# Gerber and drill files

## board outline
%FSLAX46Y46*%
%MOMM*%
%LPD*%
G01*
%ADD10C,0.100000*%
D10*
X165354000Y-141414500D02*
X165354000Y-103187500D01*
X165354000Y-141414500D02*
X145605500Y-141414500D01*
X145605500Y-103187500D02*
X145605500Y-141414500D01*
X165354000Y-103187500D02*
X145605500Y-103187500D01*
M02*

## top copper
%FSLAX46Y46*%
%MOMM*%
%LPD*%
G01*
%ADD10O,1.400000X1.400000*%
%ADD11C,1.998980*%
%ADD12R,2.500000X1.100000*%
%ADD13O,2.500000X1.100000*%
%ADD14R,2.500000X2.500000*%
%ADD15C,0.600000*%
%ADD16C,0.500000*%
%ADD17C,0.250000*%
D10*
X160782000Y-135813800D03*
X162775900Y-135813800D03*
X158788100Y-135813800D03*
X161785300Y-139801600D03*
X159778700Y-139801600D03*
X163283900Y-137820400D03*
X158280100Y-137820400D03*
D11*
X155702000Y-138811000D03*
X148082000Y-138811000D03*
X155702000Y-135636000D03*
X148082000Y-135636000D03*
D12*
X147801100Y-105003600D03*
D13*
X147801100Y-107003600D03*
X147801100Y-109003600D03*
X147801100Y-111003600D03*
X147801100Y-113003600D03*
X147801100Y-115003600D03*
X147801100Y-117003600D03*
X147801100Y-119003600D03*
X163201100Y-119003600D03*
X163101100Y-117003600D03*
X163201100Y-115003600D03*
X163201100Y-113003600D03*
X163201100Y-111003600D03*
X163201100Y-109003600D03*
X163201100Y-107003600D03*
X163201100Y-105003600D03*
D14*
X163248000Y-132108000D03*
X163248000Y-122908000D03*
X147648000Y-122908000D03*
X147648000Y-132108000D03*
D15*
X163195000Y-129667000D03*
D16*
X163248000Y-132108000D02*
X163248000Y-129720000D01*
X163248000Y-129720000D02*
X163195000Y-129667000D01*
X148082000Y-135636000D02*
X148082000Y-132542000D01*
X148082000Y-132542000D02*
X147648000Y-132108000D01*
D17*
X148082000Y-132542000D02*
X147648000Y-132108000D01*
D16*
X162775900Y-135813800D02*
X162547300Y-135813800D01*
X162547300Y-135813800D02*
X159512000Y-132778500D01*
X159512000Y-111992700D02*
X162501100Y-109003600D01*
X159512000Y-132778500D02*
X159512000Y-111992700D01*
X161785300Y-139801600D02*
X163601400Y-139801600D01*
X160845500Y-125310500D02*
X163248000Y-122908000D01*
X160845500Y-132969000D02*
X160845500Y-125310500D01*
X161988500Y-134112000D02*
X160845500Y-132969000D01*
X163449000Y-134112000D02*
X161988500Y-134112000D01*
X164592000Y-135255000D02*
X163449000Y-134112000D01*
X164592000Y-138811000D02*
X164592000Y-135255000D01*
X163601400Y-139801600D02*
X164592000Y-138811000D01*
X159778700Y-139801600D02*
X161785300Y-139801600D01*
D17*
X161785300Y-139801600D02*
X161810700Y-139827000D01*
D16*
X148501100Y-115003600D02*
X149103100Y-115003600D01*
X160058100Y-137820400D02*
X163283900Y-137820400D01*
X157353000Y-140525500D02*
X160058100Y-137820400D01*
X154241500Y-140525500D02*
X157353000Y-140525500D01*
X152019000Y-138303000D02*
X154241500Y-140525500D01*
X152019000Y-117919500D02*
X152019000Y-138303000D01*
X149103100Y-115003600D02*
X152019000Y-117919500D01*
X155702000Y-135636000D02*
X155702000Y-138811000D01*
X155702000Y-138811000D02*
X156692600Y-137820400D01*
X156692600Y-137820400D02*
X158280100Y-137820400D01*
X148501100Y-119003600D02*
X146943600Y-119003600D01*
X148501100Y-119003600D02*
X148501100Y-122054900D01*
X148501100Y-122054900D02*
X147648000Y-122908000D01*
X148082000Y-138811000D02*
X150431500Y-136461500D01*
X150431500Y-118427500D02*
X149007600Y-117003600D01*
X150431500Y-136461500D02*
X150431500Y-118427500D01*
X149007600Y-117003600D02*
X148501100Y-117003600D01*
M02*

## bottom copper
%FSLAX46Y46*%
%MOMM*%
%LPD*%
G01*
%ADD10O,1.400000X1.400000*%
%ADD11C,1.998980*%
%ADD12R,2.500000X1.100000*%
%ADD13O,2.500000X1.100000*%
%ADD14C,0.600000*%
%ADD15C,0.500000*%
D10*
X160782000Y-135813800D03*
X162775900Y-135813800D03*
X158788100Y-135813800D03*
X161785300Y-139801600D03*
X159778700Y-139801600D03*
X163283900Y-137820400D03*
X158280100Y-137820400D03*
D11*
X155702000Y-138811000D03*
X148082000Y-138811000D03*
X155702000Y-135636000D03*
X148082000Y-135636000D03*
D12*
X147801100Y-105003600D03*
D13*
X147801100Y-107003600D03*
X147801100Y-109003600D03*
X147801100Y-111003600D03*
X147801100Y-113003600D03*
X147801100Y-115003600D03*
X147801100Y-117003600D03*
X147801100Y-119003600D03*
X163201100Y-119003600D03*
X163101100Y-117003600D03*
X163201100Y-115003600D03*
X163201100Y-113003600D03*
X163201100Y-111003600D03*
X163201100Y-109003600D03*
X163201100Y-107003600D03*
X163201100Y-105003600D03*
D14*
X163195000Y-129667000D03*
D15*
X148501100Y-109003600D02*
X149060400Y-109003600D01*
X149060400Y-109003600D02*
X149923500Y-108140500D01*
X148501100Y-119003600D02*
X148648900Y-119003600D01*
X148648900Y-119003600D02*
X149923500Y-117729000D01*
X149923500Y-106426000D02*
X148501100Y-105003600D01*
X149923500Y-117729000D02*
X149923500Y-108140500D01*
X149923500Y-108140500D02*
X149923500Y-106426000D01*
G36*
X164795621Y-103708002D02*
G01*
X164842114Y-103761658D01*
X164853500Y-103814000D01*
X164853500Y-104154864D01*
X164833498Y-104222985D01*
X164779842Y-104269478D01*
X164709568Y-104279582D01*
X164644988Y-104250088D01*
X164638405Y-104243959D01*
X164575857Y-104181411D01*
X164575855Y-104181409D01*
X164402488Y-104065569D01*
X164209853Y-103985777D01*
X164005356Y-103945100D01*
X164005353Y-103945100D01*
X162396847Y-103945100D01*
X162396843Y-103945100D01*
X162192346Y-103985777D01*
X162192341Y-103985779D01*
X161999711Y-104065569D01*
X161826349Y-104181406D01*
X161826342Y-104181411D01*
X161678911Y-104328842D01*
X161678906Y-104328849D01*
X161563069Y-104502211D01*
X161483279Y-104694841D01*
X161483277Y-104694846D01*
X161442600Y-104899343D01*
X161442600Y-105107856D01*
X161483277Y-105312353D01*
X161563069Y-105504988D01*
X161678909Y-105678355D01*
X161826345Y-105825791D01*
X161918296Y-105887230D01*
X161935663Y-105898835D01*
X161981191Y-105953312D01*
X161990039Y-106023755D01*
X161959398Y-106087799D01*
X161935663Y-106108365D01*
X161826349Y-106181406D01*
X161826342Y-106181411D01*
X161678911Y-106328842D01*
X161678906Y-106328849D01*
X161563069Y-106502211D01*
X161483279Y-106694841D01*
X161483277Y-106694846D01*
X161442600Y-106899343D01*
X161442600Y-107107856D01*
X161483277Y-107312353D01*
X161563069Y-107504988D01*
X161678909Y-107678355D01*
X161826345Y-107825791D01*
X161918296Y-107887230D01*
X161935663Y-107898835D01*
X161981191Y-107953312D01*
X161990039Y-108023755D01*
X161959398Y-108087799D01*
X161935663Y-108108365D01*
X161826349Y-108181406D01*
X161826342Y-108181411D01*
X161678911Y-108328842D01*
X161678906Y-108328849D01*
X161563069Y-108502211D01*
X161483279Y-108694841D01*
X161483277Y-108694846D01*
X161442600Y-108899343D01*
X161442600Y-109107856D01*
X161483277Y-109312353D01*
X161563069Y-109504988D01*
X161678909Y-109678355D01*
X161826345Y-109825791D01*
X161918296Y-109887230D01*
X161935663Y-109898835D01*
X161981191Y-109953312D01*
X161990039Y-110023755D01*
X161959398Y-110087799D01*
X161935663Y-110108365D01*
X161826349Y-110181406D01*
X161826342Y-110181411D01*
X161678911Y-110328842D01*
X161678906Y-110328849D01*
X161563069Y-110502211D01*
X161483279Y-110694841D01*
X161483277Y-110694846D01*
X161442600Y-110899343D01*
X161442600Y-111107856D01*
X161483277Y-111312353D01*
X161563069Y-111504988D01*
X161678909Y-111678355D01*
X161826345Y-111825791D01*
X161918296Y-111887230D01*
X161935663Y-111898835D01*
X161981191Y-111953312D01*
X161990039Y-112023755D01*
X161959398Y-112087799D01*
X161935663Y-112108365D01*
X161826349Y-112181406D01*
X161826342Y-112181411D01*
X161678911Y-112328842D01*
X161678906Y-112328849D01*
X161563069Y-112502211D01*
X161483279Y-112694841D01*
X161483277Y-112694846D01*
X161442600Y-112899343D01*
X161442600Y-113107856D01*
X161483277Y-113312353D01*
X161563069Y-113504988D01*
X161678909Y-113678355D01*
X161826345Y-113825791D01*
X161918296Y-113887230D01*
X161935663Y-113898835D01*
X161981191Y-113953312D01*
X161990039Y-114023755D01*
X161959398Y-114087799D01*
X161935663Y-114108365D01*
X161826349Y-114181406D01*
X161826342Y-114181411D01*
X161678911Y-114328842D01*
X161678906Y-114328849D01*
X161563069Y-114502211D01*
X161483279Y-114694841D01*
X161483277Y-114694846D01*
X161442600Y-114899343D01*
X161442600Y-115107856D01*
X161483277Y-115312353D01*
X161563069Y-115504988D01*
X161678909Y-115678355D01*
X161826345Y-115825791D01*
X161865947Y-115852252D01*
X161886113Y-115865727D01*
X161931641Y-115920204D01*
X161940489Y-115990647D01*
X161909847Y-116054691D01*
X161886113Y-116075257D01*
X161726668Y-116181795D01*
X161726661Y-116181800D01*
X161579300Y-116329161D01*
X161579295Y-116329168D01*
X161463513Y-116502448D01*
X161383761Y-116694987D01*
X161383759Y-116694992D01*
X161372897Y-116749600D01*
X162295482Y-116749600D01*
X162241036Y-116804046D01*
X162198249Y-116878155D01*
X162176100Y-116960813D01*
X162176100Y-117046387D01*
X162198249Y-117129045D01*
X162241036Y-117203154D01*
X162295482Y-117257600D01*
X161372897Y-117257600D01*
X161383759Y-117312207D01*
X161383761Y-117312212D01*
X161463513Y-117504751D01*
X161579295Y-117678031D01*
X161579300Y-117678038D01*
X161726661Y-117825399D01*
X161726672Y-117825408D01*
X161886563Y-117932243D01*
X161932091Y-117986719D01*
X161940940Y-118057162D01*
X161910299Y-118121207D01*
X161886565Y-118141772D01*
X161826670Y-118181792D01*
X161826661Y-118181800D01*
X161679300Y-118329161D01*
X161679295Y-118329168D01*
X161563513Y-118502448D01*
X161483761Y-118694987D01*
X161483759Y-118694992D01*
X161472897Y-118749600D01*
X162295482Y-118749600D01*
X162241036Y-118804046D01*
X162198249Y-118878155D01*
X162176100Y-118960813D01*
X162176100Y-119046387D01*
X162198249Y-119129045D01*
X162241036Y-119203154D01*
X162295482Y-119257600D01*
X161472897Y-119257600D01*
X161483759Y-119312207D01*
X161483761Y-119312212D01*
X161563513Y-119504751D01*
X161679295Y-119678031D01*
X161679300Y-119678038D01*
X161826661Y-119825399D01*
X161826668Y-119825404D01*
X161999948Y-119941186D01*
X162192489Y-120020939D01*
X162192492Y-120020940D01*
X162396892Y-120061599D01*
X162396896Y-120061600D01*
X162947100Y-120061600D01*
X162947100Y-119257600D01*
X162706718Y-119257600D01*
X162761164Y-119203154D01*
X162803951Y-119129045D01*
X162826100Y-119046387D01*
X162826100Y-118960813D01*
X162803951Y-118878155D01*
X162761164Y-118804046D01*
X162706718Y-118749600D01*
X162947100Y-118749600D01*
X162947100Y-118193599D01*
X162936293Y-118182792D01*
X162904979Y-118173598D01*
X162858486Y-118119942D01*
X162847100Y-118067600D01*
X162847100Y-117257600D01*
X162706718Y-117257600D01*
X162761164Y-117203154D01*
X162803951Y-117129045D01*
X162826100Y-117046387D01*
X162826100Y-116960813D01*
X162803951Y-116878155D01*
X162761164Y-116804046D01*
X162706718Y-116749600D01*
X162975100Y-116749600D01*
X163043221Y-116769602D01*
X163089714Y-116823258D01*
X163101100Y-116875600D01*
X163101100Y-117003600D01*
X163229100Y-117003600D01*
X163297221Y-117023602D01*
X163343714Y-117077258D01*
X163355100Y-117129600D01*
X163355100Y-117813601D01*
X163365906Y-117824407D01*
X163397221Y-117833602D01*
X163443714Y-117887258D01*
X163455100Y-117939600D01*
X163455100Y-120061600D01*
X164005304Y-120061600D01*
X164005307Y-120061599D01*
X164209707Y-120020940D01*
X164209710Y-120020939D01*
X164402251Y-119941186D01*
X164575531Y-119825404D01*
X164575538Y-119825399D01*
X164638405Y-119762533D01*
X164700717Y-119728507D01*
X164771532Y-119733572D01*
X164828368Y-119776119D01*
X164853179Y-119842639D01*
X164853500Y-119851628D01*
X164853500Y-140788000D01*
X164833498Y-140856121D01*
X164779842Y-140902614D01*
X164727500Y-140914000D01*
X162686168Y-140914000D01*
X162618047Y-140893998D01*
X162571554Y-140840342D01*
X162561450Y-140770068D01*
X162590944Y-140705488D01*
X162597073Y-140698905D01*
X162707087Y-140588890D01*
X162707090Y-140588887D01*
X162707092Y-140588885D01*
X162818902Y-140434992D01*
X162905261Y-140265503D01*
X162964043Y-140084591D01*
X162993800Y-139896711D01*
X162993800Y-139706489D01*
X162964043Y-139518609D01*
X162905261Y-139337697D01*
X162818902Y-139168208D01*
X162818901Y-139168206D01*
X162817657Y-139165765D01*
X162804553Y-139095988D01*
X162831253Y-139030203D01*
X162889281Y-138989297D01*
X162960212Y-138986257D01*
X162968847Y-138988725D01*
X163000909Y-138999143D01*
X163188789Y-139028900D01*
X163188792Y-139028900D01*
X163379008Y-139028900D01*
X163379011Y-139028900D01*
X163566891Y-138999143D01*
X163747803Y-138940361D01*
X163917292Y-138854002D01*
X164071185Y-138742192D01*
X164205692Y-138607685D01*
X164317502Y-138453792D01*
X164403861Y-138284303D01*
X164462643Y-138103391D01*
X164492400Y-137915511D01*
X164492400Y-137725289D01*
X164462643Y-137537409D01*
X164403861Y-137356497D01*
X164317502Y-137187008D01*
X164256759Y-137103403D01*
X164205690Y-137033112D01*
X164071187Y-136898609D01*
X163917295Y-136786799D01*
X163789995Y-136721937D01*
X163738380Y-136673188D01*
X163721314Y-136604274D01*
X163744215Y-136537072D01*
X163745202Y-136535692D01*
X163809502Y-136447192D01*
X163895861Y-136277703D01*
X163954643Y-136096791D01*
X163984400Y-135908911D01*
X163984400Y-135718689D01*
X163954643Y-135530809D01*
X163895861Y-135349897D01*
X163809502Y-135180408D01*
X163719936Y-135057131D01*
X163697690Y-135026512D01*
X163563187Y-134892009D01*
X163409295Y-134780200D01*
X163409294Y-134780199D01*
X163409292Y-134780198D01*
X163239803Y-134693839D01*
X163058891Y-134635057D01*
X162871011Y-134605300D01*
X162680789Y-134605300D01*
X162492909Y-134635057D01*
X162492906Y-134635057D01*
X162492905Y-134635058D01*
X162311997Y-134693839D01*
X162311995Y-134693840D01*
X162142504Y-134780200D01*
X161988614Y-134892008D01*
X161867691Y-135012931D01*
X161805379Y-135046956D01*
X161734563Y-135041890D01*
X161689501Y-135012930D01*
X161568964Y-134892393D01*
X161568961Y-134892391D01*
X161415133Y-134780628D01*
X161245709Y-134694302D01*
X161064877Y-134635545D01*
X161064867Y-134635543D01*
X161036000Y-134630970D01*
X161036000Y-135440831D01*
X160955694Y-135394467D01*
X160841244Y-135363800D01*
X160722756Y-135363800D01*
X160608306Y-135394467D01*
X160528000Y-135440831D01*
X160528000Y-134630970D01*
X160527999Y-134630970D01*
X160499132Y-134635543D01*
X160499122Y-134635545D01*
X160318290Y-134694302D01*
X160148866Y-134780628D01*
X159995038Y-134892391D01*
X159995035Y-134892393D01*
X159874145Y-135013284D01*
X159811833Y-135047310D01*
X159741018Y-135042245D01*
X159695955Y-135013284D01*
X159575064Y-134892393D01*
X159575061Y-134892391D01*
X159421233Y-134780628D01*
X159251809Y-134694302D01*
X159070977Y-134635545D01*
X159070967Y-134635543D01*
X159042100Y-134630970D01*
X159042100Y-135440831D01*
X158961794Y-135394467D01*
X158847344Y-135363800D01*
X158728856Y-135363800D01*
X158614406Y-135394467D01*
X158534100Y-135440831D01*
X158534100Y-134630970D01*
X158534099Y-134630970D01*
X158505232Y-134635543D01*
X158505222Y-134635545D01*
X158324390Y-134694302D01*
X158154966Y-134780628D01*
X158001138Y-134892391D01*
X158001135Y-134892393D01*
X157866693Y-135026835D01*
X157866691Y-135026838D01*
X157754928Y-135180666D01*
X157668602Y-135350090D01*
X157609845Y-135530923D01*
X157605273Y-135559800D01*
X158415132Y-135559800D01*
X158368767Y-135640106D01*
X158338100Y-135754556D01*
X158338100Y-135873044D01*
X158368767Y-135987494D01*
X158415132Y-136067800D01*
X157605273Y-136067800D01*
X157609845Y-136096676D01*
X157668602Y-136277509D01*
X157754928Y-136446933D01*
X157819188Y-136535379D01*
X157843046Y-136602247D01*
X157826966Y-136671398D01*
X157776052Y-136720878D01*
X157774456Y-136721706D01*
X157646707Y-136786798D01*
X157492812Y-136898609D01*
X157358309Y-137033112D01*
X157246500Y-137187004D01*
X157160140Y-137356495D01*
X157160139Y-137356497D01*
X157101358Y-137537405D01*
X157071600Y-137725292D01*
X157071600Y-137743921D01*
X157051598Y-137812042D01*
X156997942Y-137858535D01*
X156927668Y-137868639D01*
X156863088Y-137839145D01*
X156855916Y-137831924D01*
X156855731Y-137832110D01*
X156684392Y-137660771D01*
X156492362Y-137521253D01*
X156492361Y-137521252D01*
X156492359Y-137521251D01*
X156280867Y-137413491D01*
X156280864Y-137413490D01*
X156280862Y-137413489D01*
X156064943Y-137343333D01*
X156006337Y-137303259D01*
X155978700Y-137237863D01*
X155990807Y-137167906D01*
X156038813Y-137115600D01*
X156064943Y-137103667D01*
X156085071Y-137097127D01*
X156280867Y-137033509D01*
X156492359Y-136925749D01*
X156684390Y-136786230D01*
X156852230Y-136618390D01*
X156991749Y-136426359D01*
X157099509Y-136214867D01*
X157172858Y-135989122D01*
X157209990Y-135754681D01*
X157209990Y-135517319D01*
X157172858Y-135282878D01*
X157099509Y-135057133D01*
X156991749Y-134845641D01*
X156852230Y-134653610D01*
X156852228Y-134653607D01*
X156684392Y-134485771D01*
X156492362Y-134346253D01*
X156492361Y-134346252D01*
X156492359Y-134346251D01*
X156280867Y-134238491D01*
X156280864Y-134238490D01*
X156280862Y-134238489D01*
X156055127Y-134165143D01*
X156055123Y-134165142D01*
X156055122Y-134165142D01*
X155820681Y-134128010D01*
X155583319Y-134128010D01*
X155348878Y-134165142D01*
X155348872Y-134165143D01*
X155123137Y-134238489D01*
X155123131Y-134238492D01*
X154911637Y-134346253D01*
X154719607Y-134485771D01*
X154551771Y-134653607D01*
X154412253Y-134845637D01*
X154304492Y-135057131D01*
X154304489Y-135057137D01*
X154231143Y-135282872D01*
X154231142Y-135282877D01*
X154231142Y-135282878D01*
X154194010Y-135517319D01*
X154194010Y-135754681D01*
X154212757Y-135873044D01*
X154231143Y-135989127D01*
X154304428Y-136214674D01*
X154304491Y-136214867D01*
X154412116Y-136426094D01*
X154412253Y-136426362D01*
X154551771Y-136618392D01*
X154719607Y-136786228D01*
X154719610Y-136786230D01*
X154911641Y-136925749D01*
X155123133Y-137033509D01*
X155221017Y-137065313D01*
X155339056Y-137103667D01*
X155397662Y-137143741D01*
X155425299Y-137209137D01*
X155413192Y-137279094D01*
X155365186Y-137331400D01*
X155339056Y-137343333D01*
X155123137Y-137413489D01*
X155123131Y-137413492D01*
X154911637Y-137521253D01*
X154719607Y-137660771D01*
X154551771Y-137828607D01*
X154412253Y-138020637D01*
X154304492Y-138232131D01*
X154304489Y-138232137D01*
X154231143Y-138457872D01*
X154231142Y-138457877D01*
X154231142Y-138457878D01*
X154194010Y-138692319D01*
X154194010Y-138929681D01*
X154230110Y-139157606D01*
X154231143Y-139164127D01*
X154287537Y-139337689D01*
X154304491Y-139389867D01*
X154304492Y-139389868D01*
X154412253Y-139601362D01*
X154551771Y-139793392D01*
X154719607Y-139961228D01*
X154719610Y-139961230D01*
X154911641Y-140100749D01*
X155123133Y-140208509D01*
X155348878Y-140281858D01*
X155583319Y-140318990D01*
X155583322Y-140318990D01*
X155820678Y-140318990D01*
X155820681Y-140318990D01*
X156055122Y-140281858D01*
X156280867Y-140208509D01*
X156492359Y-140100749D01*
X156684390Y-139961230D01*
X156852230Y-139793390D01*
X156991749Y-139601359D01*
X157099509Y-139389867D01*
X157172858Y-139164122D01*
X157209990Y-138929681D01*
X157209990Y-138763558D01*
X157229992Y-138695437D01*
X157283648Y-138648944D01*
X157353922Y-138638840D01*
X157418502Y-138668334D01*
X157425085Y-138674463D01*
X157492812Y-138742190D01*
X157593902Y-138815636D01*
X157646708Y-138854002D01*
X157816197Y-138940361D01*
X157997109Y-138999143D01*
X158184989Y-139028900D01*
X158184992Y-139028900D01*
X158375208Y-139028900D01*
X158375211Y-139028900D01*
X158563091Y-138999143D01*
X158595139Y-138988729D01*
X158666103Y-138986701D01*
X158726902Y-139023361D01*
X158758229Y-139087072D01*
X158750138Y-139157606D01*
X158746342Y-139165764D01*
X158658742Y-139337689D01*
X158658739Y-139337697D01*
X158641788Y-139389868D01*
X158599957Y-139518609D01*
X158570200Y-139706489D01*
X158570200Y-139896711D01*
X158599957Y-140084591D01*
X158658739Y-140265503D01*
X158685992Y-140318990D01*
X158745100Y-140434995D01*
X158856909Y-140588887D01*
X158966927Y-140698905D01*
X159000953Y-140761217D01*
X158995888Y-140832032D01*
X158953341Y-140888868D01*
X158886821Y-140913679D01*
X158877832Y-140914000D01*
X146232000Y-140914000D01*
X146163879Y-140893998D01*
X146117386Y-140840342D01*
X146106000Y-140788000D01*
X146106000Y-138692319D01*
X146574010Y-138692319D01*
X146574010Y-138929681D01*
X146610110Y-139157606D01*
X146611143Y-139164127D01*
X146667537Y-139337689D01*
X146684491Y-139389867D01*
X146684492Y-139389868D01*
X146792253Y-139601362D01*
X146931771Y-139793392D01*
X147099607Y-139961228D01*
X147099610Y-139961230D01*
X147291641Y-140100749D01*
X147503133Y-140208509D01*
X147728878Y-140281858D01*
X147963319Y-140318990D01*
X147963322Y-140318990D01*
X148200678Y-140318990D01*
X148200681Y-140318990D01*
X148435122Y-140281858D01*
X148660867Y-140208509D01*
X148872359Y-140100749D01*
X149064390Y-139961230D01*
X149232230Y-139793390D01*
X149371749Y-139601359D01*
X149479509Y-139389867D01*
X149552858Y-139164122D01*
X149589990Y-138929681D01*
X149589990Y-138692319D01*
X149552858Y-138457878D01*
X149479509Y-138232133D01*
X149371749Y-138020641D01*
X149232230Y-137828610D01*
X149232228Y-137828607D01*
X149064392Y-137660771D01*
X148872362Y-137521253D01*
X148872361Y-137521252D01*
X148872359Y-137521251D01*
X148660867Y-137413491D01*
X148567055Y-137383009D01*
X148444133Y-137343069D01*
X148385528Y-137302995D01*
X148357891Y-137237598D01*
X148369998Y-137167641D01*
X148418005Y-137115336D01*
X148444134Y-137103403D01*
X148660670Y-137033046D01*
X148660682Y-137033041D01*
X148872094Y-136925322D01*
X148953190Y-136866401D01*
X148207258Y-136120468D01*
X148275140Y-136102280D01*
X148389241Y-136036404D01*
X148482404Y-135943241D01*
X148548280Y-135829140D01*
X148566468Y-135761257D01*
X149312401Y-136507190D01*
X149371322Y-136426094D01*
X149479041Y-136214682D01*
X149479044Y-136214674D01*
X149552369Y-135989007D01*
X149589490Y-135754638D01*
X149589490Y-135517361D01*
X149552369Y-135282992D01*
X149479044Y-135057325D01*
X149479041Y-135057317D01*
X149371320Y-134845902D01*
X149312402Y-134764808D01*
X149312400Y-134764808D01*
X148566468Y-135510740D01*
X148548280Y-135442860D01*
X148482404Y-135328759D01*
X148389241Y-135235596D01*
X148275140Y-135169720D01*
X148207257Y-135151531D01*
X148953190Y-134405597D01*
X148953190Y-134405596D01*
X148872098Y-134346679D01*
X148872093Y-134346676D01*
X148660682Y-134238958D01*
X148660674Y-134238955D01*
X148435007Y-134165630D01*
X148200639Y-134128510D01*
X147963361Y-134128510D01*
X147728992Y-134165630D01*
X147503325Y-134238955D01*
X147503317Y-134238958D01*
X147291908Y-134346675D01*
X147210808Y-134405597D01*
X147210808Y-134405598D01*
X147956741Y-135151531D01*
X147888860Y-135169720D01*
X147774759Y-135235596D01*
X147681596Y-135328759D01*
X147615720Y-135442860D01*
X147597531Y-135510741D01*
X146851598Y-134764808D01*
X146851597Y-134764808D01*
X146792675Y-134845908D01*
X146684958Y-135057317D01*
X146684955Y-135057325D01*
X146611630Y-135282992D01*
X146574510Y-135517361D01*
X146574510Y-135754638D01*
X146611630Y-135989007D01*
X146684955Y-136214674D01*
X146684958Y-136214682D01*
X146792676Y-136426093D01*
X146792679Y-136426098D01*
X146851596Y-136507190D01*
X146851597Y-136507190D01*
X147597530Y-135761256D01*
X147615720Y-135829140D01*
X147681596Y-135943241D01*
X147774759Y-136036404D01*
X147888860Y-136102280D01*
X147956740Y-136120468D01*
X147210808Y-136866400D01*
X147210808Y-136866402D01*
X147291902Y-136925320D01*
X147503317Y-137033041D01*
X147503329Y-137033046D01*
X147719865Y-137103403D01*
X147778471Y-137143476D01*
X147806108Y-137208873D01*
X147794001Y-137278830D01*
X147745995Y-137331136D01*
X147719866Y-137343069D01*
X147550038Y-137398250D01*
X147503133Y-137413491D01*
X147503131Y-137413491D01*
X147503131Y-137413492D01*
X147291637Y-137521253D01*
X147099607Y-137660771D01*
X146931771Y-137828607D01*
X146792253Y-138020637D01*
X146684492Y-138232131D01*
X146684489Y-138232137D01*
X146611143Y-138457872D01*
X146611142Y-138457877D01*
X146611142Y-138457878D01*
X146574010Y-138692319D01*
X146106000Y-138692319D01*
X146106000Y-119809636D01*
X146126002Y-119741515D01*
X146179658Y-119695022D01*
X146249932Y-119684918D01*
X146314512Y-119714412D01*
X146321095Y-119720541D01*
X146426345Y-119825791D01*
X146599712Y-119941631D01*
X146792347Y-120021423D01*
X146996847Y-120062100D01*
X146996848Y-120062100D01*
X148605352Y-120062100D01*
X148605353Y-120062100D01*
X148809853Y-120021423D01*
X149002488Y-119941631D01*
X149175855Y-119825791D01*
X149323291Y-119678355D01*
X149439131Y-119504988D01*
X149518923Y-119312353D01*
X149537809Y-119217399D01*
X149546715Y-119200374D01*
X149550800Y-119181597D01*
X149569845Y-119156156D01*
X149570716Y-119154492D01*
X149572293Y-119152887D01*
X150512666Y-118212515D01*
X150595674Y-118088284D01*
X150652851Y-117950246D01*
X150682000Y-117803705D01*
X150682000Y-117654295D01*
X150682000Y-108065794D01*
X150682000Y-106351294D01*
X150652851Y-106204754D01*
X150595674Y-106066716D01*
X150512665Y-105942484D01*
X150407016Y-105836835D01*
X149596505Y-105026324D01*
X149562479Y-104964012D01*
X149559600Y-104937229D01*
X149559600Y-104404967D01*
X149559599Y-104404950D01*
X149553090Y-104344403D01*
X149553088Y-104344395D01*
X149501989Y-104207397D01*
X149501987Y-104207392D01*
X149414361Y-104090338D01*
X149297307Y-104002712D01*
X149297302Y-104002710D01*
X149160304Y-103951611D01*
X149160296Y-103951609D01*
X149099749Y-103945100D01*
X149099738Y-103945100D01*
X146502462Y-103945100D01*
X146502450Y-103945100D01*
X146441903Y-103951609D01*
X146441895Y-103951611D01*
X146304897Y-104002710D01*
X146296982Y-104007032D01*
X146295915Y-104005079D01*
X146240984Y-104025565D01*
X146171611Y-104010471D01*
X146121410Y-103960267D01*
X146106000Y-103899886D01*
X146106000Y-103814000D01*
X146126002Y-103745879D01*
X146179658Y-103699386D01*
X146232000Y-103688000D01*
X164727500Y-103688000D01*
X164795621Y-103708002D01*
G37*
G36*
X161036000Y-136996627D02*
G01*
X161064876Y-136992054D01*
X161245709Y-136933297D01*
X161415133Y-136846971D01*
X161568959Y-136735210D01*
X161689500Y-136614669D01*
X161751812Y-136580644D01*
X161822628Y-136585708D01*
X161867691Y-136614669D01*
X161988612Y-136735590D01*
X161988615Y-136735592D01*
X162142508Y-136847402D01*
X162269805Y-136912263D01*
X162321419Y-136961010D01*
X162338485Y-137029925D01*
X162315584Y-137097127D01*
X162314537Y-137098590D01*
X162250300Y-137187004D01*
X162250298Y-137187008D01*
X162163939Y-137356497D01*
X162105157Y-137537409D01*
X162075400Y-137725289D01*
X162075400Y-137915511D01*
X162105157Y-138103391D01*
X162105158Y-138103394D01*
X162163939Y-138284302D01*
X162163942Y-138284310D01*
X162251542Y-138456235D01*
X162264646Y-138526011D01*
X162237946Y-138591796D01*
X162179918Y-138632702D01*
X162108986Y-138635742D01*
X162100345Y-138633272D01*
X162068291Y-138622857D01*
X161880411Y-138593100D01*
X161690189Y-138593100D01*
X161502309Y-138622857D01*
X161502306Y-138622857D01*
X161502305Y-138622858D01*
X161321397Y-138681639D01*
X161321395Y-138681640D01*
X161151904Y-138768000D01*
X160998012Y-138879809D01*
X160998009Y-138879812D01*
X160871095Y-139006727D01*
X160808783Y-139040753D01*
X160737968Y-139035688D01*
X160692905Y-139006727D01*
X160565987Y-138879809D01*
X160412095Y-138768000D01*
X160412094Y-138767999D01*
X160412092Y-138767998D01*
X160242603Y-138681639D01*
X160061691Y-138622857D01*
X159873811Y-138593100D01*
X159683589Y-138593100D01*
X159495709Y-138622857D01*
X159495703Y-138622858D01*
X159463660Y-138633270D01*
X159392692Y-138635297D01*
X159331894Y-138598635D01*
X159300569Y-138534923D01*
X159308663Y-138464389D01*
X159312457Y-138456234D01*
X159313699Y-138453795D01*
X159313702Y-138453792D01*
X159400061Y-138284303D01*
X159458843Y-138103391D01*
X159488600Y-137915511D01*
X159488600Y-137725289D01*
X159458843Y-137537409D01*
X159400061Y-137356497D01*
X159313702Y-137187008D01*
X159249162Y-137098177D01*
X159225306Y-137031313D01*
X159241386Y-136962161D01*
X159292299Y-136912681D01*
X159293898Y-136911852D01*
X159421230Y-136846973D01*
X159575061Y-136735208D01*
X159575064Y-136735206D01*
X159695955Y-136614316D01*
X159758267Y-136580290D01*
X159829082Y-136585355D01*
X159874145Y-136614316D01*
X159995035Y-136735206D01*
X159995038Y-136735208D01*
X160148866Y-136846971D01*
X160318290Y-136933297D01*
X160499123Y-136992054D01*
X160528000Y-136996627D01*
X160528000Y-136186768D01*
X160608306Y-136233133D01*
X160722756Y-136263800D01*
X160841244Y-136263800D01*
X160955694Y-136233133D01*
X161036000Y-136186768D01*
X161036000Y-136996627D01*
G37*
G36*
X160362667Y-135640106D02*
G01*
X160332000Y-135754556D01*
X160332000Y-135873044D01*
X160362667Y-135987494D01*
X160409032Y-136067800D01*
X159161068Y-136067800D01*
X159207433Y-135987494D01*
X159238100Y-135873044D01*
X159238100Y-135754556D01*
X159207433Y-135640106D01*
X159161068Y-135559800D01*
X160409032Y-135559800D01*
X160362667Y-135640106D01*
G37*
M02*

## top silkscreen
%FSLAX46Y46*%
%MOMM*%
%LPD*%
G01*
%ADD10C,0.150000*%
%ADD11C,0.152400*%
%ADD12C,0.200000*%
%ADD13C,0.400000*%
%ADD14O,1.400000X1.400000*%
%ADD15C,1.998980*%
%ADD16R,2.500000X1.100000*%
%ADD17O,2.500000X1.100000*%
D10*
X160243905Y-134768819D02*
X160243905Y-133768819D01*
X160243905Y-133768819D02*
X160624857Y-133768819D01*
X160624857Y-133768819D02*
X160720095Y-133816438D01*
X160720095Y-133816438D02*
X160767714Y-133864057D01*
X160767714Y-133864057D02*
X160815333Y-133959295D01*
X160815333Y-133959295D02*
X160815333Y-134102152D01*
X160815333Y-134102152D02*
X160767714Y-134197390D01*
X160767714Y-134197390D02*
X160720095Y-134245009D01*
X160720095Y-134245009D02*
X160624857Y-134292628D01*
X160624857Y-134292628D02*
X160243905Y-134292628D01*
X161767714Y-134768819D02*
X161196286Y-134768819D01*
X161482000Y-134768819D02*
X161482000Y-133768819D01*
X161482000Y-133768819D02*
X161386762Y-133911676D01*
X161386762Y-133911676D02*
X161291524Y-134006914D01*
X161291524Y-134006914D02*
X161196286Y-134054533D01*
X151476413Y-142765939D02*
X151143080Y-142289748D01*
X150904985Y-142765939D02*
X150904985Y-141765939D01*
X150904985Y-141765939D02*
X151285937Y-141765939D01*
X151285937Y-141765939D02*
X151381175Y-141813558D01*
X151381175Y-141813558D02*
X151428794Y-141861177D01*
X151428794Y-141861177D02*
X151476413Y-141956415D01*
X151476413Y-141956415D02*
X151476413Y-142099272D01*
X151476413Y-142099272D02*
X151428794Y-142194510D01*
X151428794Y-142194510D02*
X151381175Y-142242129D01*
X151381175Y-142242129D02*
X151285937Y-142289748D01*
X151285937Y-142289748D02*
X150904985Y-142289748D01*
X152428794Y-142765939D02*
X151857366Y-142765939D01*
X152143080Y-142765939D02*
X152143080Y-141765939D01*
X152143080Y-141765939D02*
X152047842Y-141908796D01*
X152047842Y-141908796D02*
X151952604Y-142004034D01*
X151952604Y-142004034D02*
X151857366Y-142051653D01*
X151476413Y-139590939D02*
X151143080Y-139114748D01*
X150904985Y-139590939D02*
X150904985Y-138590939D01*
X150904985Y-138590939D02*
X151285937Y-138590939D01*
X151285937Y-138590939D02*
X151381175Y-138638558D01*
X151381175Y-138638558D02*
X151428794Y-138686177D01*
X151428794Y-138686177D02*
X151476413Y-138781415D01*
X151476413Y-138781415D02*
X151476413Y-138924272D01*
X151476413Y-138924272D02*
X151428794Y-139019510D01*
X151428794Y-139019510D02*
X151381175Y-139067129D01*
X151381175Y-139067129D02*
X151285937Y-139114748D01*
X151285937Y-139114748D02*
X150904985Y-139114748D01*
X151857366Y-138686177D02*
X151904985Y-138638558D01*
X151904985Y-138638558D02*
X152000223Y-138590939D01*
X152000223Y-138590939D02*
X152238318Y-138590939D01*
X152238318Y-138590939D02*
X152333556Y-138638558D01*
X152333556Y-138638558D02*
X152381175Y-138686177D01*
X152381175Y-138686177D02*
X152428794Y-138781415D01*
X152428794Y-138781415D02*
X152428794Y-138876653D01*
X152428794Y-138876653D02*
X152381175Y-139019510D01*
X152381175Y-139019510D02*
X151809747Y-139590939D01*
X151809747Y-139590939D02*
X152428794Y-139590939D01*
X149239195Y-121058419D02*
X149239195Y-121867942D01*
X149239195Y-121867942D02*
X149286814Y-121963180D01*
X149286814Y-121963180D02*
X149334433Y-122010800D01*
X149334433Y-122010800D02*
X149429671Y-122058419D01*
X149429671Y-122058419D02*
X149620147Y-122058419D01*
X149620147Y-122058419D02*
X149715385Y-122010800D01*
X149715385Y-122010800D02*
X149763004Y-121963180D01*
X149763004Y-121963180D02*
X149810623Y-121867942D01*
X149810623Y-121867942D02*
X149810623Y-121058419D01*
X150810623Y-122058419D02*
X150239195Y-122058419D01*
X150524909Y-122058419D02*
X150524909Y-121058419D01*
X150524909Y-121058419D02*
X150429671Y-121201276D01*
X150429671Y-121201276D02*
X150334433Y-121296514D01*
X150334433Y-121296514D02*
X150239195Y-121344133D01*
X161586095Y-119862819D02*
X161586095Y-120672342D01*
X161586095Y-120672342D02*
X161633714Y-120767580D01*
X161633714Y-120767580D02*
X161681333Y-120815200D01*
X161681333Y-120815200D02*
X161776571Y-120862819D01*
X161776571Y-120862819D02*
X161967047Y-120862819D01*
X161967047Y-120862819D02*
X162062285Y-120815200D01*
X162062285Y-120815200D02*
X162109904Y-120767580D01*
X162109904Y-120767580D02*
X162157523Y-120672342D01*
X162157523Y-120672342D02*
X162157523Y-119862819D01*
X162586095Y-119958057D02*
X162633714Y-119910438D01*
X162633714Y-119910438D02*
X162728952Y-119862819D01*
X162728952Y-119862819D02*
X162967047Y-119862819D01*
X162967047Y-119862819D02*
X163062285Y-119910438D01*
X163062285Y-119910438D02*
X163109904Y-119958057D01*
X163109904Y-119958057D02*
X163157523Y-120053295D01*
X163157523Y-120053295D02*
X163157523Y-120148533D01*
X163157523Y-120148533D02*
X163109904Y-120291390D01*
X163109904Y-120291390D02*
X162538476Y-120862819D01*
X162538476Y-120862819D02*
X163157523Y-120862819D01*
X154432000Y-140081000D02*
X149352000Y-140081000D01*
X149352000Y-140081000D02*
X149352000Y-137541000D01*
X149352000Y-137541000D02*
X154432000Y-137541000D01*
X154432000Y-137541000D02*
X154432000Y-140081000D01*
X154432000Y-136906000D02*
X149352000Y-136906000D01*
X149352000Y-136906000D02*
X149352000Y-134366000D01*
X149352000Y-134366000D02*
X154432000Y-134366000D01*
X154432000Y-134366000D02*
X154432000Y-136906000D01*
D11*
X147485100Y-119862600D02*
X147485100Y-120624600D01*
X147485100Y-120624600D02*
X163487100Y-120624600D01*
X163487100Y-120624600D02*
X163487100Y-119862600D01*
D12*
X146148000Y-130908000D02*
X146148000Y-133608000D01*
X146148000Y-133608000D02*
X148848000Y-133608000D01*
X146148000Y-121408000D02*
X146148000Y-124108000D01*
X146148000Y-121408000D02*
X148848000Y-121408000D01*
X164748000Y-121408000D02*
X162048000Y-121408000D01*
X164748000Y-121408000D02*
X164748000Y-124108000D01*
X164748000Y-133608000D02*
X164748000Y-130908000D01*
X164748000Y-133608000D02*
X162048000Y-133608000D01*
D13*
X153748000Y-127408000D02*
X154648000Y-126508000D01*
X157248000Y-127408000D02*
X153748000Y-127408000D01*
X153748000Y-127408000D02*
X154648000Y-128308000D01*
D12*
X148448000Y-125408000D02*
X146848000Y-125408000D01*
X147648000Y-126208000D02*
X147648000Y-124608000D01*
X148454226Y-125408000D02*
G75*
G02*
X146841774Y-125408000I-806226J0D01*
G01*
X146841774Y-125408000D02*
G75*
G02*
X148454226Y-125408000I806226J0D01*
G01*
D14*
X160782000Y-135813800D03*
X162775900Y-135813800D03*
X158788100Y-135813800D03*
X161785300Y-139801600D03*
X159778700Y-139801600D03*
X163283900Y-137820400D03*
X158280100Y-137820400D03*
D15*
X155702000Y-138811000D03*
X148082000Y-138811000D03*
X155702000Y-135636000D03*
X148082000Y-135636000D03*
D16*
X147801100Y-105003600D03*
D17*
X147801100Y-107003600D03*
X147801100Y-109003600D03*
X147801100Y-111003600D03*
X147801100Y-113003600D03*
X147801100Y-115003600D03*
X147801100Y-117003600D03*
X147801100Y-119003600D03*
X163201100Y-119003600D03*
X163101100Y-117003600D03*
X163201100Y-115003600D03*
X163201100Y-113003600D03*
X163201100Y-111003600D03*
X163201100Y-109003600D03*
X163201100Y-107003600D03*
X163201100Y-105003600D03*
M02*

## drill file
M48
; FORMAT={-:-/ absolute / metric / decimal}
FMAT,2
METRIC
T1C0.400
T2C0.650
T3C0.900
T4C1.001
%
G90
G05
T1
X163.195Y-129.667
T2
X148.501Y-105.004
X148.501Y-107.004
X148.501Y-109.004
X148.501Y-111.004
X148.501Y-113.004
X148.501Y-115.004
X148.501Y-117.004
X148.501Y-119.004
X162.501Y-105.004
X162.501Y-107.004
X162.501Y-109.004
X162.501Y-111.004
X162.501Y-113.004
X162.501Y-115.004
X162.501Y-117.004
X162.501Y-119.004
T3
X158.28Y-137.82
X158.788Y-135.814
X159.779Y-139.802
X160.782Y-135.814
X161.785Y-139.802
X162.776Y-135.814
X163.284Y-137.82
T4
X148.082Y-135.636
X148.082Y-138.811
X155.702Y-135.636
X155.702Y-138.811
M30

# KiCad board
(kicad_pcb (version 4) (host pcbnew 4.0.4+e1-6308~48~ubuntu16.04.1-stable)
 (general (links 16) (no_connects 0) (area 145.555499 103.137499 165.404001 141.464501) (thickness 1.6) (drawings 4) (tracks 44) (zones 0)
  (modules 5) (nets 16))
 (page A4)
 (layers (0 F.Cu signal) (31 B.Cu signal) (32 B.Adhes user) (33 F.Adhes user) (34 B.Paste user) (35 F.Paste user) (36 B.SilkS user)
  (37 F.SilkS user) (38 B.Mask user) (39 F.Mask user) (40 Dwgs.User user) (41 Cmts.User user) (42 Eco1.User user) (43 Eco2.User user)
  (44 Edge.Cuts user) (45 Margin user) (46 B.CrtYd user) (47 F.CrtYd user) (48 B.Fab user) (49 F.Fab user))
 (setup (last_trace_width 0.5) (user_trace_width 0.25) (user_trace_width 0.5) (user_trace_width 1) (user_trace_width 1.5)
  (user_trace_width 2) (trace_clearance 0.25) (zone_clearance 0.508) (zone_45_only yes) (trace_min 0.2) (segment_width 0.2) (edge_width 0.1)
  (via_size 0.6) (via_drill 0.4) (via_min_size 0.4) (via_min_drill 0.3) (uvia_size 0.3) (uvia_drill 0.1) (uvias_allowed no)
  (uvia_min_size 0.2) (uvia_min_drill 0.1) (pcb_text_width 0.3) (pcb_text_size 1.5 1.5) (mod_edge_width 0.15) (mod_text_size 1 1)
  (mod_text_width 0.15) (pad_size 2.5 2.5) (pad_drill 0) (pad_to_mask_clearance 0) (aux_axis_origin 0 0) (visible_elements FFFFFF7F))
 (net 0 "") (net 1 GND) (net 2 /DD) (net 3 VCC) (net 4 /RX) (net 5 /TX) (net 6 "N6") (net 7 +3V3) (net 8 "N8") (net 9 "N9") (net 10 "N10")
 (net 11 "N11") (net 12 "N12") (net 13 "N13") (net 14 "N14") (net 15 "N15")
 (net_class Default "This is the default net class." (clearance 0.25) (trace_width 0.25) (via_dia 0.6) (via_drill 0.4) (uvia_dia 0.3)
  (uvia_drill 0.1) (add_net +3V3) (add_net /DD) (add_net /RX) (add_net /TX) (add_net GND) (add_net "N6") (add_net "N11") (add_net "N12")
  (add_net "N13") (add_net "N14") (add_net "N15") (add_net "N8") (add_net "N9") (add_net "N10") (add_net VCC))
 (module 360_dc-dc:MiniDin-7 (layer F.Cu) (at 160.782 137.414)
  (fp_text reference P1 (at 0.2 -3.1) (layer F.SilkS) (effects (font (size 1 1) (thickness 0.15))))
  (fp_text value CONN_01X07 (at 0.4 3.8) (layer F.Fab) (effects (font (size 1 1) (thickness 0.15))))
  (pad 6 thru_hole oval (at 0 -1.6002) (size 1.4 1.4) (drill oval 0.9) (layers *.Cu *.Mask F.SilkS) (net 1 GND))
  (pad 5 thru_hole oval (at 1.9939 -1.6002) (size 1.4 1.4) (drill oval 0.9) (layers *.Cu *.Mask F.SilkS) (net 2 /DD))
  (pad 7 thru_hole oval (at -1.9939 -1.6002) (size 1.4 1.4) (drill oval 0.9) (layers *.Cu *.Mask F.SilkS) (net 1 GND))
  (pad 1 thru_hole oval (at 1.0033 2.3876) (size 1.4 1.4) (drill oval 0.9) (layers *.Cu *.Mask F.SilkS) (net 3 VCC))
  (pad 2 thru_hole oval (at -1.0033 2.3876) (size 1.4 1.4) (drill oval 0.9) (layers *.Cu *.Mask F.SilkS) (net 3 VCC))
  (pad 3 thru_hole oval (at 2.5019 0.4064) (size 1.4 1.4) (drill oval 0.9) (layers *.Cu *.Mask F.SilkS) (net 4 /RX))
  (pad 4 thru_hole oval (at -2.5019 0.4064) (size 1.4 1.4) (drill oval 0.9) (layers *.Cu *.Mask F.SilkS) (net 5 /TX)))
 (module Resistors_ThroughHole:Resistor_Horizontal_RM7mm (layer F.Cu) (at 155.702 138.811 180)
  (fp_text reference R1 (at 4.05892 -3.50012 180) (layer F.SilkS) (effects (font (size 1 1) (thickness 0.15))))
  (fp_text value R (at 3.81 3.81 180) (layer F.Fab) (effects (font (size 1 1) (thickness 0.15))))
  (fp_line (start 1.27 -1.27) (end 6.35 -1.27) (layer F.SilkS) (width 0.15))
  (fp_line (start 6.35 -1.27) (end 6.35 1.27) (layer F.SilkS) (width 0.15))
  (fp_line (start 6.35 1.27) (end 1.27 1.27) (layer F.SilkS) (width 0.15))
  (fp_line (start 1.27 1.27) (end 1.27 -1.27) (layer F.SilkS) (width 0.15))
  (pad 1 thru_hole circle (at 0 0 180) (size 1.99898 1.99898) (drill 1.00076) (layers *.Cu *.SilkS *.Mask) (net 5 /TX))
  (pad 2 thru_hole circle (at 7.62 0 180) (size 1.99898 1.99898) (drill 1.00076) (layers *.Cu *.SilkS *.Mask) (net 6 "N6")))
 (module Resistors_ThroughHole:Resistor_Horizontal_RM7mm (layer F.Cu) (at 155.702 135.636 180)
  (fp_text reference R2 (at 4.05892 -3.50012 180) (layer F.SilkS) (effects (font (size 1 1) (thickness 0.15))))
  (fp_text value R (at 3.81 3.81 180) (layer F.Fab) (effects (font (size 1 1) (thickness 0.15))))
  (fp_line (start 1.27 -1.27) (end 6.35 -1.27) (layer F.SilkS) (width 0.15))
  (fp_line (start 6.35 -1.27) (end 6.35 1.27) (layer F.SilkS) (width 0.15))
  (fp_line (start 6.35 1.27) (end 1.27 1.27) (layer F.SilkS) (width 0.15))
  (fp_line (start 1.27 1.27) (end 1.27 -1.27) (layer F.SilkS) (width 0.15))
  (pad 1 thru_hole circle (at 0 0 180) (size 1.99898 1.99898) (drill 1.00076) (layers *.Cu *.SilkS *.Mask) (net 5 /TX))
  (pad 2 thru_hole circle (at 7.62 0 180) (size 1.99898 1.99898) (drill 1.00076) (layers *.Cu *.SilkS *.Mask) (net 1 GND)))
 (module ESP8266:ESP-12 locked (layer F.Cu) (at 148.5011 105.0036)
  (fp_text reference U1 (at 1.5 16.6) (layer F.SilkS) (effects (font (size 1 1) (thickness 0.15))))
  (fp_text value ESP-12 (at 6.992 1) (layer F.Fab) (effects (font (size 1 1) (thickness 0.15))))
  (fp_line (start -1.016 14.859) (end -1.016 15.621) (layer F.SilkS) (width 0.1524))
  (fp_line (start -1.016 15.621) (end 14.986 15.621) (layer F.SilkS) (width 0.1524))
  (fp_line (start 14.986 15.621) (end 14.986 14.859) (layer F.SilkS) (width 0.1524))
  (pad 1 thru_hole rect (at 0 0) (size 2.5 1.1) (drill 0.65 (offset -0.7 0)) (layers *.Cu *.Mask F.SilkS) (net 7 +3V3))
  (pad 2 thru_hole oval (at 0 2) (size 2.5 1.1) (drill 0.65 (offset -0.7 0)) (layers *.Cu *.Mask F.SilkS) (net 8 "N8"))
  (pad 3 thru_hole oval (at 0 4) (size 2.5 1.1) (drill 0.65 (offset -0.7 0)) (layers *.Cu *.Mask F.SilkS) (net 7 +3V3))
  (pad 4 thru_hole oval (at 0 6) (size 2.5 1.1) (drill 0.65 (offset -0.7 0)) (layers *.Cu *.Mask F.SilkS) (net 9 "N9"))
  (pad 5 thru_hole oval (at 0 8) (size 2.5 1.1) (drill 0.65 (offset -0.7 0)) (layers *.Cu *.Mask F.SilkS) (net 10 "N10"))
  (pad 6 thru_hole oval (at 0 10) (size 2.5 1.1) (drill 0.65 (offset -0.7 0)) (layers *.Cu *.Mask F.SilkS) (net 4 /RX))
  (pad 7 thru_hole oval (at 0 12) (size 2.5 1.1) (drill 0.65 (offset -0.7 0)) (layers *.Cu *.Mask F.SilkS) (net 6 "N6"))
  (pad 8 thru_hole oval (at 0 14) (size 2.5 1.1) (drill 0.65 (offset -0.7 0)) (layers *.Cu *.Mask F.SilkS) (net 7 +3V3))
  (pad 9 thru_hole oval (at 14 14) (size 2.5 1.1) (drill 0.65 (offset 0.7 0)) (layers *.Cu *.Mask F.SilkS) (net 1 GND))
  (pad 10 thru_hole oval (at 14 12) (size 2.5 1.1) (drill 0.65 (offset 0.6 0)) (layers *.Cu *.Mask F.SilkS) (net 1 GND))
  (pad 11 thru_hole oval (at 14 10) (size 2.5 1.1) (drill 0.65 (offset 0.7 0)) (layers *.Cu *.Mask F.SilkS) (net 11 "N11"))
  (pad 12 thru_hole oval (at 14 8) (size 2.5 1.1) (drill 0.65 (offset 0.7 0)) (layers *.Cu *.Mask F.SilkS) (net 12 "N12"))
  (pad 13 thru_hole oval (at 14 6) (size 2.5 1.1) (drill 0.65 (offset 0.7 0)) (layers *.Cu *.Mask F.SilkS) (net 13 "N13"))
  (pad 14 thru_hole oval (at 14 4) (size 2.5 1.1) (drill 0.65 (offset 0.7 0)) (layers *.Cu *.Mask F.SilkS) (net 2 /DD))
  (pad 15 thru_hole oval (at 14 2) (size 2.5 1.1) (drill 0.65 (offset 0.7 0)) (layers *.Cu *.Mask F.SilkS) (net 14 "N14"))
  (pad 16 thru_hole oval (at 14 0) (size 2.5 1.1) (drill 0.65 (offset 0.7 0)) (layers *.Cu *.Mask F.SilkS) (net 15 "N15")))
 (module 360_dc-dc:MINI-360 (layer F.Cu) (at 155.448 127.508 180)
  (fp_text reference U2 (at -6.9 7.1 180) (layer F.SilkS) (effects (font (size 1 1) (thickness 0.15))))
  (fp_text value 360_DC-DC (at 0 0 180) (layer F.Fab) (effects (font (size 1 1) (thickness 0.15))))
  (fp_line (start 9.3 -3.4) (end 9.3 -6.1) (layer F.SilkS) (width 0.2))
  (fp_line (start 9.3 -6.1) (end 6.6 -6.1) (layer F.SilkS) (width 0.2))
  (fp_line (start 9.3 6.1) (end 9.3 3.4) (layer F.SilkS) (width 0.2))
  (fp_line (start 9.3 6.1) (end 6.6 6.1) (layer F.SilkS) (width 0.2))
  (fp_line (start -9.3 6.1) (end -6.6 6.1) (layer F.SilkS) (width 0.2))
  (fp_line (start -9.3 6.1) (end -9.3 3.4) (layer F.SilkS) (width 0.2))
  (fp_line (start -9.3 -6.1) (end -9.3 -3.4) (layer F.SilkS) (width 0.2))
  (fp_line (start -9.3 -6.1) (end -6.6 -6.1) (layer F.SilkS) (width 0.2))
  (fp_line (start 1.7 0.1) (end 0.8 1) (layer F.SilkS) (width 0.4))
  (fp_line (start -1.8 0.1) (end 1.7 0.1) (layer F.SilkS) (width 0.4))
  (fp_line (start 1.7 0.1) (end 0.8 -0.8) (layer F.SilkS) (width 0.4))
  (fp_line (start 7 2.1) (end 8.6 2.1) (layer F.SilkS) (width 0.2))
  (fp_line (start 7.8 1.3) (end 7.8 2.9) (layer F.SilkS) (width 0.2))
  (fp_circle (center 7.8 2.1) (end 7.9 2.9) (layer F.SilkS) (width 0.2))
  (pad GND smd rect (at -7.8 -4.6 180) (size 2.5 2.5) (layers F.Cu F.Paste F.Mask) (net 1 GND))
  (pad VIN smd rect (at -7.8 4.6 180) (size 2.5 2.5) (layers F.Cu F.Paste F.Mask) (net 3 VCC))
  (pad VOUT smd rect (at 7.8 4.6 180) (size 2.5 2.5) (layers F.Cu F.Paste F.Mask) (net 7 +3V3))
  (pad GND smd rect (at 7.8 -4.6 180) (size 2.5 2.5) (layers F.Cu F.Paste F.Mask) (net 1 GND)))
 (gr_line (start 165.354 141.4145) (end 165.354 103.1875) (angle 90) (layer Edge.Cuts) (width 0.1))
 (gr_line (start 165.354 141.4145) (end 145.6055 141.4145) (angle 90) (layer Edge.Cuts) (width 0.1))
 (gr_line (start 145.6055 103.1875) (end 145.6055 141.4145) (angle 90) (layer Edge.Cuts) (width 0.1))
 (gr_line (start 165.354 103.1875) (end 145.6055 103.1875) (angle 90) (layer Edge.Cuts) (width 0.1))
 (segment (start 163.248 132.108) (end 163.248 129.72) (width 0.5) (layer F.Cu) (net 1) (status 400000))
 (via (at 163.195 129.667) (size 0.6) (drill 0.4) (layers F.Cu B.Cu) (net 1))
 (segment (start 163.248 129.72) (end 163.195 129.667) (width 0.5) (layer F.Cu) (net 1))
 (segment (start 148.082 135.636) (end 148.082 132.542) (width 0.5) (layer F.Cu) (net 1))
 (segment (start 148.082 132.542) (end 147.648 132.108) (width 0.5) (layer F.Cu) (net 1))
 (segment (start 148.082 132.542) (end 147.648 132.108) (width 0.25) (layer F.Cu) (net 1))
 (segment (start 162.7759 135.8138) (end 162.5473 135.8138) (width 0.5) (layer F.Cu) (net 2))
 (segment (start 162.5473 135.8138) (end 159.512 132.7785) (width 0.5) (layer F.Cu) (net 2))
 (segment (start 159.512 111.9927) (end 162.5011 109.0036) (width 0.5) (layer F.Cu) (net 2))
 (segment (start 159.512 132.7785) (end 159.512 111.9927) (width 0.5) (layer F.Cu) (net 2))
 (segment (start 161.7853 139.8016) (end 163.6014 139.8016) (width 0.5) (layer F.Cu) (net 3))
 (segment (start 160.8455 125.3105) (end 163.248 122.908) (width 0.5) (layer F.Cu) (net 3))
 (segment (start 160.8455 132.969) (end 160.8455 125.3105) (width 0.5) (layer F.Cu) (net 3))
 (segment (start 161.9885 134.112) (end 160.8455 132.969) (width 0.5) (layer F.Cu) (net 3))
 (segment (start 163.449 134.112) (end 161.9885 134.112) (width 0.5) (layer F.Cu) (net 3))
 (segment (start 164.592 135.255) (end 163.449 134.112) (width 0.5) (layer F.Cu) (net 3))
 (segment (start 164.592 138.811) (end 164.592 135.255) (width 0.5) (layer F.Cu) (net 3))
 (segment (start 163.6014 139.8016) (end 164.592 138.811) (width 0.5) (layer F.Cu) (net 3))
 (segment (start 159.7787 139.8016) (end 161.7853 139.8016) (width 0.5) (layer F.Cu) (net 3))
 (segment (start 161.7853 139.8016) (end 161.8107 139.827) (width 0.25) (layer F.Cu) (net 3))
 (segment (start 148.5011 115.0036) (end 149.1031 115.0036) (width 0.5) (layer F.Cu) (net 4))
 (segment (start 160.0581 137.8204) (end 163.2839 137.8204) (width 0.5) (layer F.Cu) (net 4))
 (segment (start 157.353 140.5255) (end 160.0581 137.8204) (width 0.5) (layer F.Cu) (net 4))
 (segment (start 154.2415 140.5255) (end 157.353 140.5255) (width 0.5) (layer F.Cu) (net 4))
 (segment (start 152.019 138.303) (end 154.2415 140.5255) (width 0.5) (layer F.Cu) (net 4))
 (segment (start 152.019 117.9195) (end 152.019 138.303) (width 0.5) (layer F.Cu) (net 4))
 (segment (start 149.1031 115.0036) (end 152.019 117.9195) (width 0.5) (layer F.Cu) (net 4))
 (segment (start 155.702 135.636) (end 155.702 138.811) (width 0.5) (layer F.Cu) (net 5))
 (segment (start 155.702 138.811) (end 156.6926 137.8204) (width 0.5) (layer F.Cu) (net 5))
 (segment (start 156.6926 137.8204) (end 158.2801 137.8204) (width 0.5) (layer F.Cu) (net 5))
 (segment (start 148.5011 109.0036) (end 149.0604 109.0036) (width 0.5) (layer B.Cu) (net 7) (status 400000))
 (segment (start 149.0604 109.0036) (end 149.9235 108.1405) (width 0.5) (layer B.Cu) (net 7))
 (segment (start 148.5011 119.0036) (end 148.6489 119.0036) (width 0.5) (layer B.Cu) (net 7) (status C00000))
 (segment (start 148.6489 119.0036) (end 149.9235 117.729) (width 0.5) (layer B.Cu) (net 7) (status 400000))
 (segment (start 149.9235 106.426) (end 148.5011 105.0036) (width 0.5) (layer B.Cu) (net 7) (status 800000))
 (segment (start 149.9235 117.729) (end 149.9235 108.1405) (width 0.5) (layer B.Cu) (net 7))
 (segment (start 149.9235 108.1405) (end 149.9235 106.426) (width 0.5) (layer B.Cu) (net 7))
 (segment (start 148.5011 119.0036) (end 146.9436 119.0036) (width 0.5) (layer F.Cu) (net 7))
 (segment (start 148.5011 119.0036) (end 148.5011 122.0549) (width 0.5) (layer F.Cu) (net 7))
 (segment (start 148.5011 122.0549) (end 147.648 122.908) (width 0.5) (layer F.Cu) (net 7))
 (segment (start 148.082 138.811) (end 150.4315 136.4615) (width 0.5) (layer F.Cu) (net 6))
 (segment (start 150.4315 118.4275) (end 149.0076 117.0036) (width 0.5) (layer F.Cu) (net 6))
 (segment (start 150.4315 136.4615) (end 150.4315 118.4275) (width 0.5) (layer F.Cu) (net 6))
 (segment (start 149.0076 117.0036) (end 148.5011 117.0036) (width 0.5) (layer F.Cu) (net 6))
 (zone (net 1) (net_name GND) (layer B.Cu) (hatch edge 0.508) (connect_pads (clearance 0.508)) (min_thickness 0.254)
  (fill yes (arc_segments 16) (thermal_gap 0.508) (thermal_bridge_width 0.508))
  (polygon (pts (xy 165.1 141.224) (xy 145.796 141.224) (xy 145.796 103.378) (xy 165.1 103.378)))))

